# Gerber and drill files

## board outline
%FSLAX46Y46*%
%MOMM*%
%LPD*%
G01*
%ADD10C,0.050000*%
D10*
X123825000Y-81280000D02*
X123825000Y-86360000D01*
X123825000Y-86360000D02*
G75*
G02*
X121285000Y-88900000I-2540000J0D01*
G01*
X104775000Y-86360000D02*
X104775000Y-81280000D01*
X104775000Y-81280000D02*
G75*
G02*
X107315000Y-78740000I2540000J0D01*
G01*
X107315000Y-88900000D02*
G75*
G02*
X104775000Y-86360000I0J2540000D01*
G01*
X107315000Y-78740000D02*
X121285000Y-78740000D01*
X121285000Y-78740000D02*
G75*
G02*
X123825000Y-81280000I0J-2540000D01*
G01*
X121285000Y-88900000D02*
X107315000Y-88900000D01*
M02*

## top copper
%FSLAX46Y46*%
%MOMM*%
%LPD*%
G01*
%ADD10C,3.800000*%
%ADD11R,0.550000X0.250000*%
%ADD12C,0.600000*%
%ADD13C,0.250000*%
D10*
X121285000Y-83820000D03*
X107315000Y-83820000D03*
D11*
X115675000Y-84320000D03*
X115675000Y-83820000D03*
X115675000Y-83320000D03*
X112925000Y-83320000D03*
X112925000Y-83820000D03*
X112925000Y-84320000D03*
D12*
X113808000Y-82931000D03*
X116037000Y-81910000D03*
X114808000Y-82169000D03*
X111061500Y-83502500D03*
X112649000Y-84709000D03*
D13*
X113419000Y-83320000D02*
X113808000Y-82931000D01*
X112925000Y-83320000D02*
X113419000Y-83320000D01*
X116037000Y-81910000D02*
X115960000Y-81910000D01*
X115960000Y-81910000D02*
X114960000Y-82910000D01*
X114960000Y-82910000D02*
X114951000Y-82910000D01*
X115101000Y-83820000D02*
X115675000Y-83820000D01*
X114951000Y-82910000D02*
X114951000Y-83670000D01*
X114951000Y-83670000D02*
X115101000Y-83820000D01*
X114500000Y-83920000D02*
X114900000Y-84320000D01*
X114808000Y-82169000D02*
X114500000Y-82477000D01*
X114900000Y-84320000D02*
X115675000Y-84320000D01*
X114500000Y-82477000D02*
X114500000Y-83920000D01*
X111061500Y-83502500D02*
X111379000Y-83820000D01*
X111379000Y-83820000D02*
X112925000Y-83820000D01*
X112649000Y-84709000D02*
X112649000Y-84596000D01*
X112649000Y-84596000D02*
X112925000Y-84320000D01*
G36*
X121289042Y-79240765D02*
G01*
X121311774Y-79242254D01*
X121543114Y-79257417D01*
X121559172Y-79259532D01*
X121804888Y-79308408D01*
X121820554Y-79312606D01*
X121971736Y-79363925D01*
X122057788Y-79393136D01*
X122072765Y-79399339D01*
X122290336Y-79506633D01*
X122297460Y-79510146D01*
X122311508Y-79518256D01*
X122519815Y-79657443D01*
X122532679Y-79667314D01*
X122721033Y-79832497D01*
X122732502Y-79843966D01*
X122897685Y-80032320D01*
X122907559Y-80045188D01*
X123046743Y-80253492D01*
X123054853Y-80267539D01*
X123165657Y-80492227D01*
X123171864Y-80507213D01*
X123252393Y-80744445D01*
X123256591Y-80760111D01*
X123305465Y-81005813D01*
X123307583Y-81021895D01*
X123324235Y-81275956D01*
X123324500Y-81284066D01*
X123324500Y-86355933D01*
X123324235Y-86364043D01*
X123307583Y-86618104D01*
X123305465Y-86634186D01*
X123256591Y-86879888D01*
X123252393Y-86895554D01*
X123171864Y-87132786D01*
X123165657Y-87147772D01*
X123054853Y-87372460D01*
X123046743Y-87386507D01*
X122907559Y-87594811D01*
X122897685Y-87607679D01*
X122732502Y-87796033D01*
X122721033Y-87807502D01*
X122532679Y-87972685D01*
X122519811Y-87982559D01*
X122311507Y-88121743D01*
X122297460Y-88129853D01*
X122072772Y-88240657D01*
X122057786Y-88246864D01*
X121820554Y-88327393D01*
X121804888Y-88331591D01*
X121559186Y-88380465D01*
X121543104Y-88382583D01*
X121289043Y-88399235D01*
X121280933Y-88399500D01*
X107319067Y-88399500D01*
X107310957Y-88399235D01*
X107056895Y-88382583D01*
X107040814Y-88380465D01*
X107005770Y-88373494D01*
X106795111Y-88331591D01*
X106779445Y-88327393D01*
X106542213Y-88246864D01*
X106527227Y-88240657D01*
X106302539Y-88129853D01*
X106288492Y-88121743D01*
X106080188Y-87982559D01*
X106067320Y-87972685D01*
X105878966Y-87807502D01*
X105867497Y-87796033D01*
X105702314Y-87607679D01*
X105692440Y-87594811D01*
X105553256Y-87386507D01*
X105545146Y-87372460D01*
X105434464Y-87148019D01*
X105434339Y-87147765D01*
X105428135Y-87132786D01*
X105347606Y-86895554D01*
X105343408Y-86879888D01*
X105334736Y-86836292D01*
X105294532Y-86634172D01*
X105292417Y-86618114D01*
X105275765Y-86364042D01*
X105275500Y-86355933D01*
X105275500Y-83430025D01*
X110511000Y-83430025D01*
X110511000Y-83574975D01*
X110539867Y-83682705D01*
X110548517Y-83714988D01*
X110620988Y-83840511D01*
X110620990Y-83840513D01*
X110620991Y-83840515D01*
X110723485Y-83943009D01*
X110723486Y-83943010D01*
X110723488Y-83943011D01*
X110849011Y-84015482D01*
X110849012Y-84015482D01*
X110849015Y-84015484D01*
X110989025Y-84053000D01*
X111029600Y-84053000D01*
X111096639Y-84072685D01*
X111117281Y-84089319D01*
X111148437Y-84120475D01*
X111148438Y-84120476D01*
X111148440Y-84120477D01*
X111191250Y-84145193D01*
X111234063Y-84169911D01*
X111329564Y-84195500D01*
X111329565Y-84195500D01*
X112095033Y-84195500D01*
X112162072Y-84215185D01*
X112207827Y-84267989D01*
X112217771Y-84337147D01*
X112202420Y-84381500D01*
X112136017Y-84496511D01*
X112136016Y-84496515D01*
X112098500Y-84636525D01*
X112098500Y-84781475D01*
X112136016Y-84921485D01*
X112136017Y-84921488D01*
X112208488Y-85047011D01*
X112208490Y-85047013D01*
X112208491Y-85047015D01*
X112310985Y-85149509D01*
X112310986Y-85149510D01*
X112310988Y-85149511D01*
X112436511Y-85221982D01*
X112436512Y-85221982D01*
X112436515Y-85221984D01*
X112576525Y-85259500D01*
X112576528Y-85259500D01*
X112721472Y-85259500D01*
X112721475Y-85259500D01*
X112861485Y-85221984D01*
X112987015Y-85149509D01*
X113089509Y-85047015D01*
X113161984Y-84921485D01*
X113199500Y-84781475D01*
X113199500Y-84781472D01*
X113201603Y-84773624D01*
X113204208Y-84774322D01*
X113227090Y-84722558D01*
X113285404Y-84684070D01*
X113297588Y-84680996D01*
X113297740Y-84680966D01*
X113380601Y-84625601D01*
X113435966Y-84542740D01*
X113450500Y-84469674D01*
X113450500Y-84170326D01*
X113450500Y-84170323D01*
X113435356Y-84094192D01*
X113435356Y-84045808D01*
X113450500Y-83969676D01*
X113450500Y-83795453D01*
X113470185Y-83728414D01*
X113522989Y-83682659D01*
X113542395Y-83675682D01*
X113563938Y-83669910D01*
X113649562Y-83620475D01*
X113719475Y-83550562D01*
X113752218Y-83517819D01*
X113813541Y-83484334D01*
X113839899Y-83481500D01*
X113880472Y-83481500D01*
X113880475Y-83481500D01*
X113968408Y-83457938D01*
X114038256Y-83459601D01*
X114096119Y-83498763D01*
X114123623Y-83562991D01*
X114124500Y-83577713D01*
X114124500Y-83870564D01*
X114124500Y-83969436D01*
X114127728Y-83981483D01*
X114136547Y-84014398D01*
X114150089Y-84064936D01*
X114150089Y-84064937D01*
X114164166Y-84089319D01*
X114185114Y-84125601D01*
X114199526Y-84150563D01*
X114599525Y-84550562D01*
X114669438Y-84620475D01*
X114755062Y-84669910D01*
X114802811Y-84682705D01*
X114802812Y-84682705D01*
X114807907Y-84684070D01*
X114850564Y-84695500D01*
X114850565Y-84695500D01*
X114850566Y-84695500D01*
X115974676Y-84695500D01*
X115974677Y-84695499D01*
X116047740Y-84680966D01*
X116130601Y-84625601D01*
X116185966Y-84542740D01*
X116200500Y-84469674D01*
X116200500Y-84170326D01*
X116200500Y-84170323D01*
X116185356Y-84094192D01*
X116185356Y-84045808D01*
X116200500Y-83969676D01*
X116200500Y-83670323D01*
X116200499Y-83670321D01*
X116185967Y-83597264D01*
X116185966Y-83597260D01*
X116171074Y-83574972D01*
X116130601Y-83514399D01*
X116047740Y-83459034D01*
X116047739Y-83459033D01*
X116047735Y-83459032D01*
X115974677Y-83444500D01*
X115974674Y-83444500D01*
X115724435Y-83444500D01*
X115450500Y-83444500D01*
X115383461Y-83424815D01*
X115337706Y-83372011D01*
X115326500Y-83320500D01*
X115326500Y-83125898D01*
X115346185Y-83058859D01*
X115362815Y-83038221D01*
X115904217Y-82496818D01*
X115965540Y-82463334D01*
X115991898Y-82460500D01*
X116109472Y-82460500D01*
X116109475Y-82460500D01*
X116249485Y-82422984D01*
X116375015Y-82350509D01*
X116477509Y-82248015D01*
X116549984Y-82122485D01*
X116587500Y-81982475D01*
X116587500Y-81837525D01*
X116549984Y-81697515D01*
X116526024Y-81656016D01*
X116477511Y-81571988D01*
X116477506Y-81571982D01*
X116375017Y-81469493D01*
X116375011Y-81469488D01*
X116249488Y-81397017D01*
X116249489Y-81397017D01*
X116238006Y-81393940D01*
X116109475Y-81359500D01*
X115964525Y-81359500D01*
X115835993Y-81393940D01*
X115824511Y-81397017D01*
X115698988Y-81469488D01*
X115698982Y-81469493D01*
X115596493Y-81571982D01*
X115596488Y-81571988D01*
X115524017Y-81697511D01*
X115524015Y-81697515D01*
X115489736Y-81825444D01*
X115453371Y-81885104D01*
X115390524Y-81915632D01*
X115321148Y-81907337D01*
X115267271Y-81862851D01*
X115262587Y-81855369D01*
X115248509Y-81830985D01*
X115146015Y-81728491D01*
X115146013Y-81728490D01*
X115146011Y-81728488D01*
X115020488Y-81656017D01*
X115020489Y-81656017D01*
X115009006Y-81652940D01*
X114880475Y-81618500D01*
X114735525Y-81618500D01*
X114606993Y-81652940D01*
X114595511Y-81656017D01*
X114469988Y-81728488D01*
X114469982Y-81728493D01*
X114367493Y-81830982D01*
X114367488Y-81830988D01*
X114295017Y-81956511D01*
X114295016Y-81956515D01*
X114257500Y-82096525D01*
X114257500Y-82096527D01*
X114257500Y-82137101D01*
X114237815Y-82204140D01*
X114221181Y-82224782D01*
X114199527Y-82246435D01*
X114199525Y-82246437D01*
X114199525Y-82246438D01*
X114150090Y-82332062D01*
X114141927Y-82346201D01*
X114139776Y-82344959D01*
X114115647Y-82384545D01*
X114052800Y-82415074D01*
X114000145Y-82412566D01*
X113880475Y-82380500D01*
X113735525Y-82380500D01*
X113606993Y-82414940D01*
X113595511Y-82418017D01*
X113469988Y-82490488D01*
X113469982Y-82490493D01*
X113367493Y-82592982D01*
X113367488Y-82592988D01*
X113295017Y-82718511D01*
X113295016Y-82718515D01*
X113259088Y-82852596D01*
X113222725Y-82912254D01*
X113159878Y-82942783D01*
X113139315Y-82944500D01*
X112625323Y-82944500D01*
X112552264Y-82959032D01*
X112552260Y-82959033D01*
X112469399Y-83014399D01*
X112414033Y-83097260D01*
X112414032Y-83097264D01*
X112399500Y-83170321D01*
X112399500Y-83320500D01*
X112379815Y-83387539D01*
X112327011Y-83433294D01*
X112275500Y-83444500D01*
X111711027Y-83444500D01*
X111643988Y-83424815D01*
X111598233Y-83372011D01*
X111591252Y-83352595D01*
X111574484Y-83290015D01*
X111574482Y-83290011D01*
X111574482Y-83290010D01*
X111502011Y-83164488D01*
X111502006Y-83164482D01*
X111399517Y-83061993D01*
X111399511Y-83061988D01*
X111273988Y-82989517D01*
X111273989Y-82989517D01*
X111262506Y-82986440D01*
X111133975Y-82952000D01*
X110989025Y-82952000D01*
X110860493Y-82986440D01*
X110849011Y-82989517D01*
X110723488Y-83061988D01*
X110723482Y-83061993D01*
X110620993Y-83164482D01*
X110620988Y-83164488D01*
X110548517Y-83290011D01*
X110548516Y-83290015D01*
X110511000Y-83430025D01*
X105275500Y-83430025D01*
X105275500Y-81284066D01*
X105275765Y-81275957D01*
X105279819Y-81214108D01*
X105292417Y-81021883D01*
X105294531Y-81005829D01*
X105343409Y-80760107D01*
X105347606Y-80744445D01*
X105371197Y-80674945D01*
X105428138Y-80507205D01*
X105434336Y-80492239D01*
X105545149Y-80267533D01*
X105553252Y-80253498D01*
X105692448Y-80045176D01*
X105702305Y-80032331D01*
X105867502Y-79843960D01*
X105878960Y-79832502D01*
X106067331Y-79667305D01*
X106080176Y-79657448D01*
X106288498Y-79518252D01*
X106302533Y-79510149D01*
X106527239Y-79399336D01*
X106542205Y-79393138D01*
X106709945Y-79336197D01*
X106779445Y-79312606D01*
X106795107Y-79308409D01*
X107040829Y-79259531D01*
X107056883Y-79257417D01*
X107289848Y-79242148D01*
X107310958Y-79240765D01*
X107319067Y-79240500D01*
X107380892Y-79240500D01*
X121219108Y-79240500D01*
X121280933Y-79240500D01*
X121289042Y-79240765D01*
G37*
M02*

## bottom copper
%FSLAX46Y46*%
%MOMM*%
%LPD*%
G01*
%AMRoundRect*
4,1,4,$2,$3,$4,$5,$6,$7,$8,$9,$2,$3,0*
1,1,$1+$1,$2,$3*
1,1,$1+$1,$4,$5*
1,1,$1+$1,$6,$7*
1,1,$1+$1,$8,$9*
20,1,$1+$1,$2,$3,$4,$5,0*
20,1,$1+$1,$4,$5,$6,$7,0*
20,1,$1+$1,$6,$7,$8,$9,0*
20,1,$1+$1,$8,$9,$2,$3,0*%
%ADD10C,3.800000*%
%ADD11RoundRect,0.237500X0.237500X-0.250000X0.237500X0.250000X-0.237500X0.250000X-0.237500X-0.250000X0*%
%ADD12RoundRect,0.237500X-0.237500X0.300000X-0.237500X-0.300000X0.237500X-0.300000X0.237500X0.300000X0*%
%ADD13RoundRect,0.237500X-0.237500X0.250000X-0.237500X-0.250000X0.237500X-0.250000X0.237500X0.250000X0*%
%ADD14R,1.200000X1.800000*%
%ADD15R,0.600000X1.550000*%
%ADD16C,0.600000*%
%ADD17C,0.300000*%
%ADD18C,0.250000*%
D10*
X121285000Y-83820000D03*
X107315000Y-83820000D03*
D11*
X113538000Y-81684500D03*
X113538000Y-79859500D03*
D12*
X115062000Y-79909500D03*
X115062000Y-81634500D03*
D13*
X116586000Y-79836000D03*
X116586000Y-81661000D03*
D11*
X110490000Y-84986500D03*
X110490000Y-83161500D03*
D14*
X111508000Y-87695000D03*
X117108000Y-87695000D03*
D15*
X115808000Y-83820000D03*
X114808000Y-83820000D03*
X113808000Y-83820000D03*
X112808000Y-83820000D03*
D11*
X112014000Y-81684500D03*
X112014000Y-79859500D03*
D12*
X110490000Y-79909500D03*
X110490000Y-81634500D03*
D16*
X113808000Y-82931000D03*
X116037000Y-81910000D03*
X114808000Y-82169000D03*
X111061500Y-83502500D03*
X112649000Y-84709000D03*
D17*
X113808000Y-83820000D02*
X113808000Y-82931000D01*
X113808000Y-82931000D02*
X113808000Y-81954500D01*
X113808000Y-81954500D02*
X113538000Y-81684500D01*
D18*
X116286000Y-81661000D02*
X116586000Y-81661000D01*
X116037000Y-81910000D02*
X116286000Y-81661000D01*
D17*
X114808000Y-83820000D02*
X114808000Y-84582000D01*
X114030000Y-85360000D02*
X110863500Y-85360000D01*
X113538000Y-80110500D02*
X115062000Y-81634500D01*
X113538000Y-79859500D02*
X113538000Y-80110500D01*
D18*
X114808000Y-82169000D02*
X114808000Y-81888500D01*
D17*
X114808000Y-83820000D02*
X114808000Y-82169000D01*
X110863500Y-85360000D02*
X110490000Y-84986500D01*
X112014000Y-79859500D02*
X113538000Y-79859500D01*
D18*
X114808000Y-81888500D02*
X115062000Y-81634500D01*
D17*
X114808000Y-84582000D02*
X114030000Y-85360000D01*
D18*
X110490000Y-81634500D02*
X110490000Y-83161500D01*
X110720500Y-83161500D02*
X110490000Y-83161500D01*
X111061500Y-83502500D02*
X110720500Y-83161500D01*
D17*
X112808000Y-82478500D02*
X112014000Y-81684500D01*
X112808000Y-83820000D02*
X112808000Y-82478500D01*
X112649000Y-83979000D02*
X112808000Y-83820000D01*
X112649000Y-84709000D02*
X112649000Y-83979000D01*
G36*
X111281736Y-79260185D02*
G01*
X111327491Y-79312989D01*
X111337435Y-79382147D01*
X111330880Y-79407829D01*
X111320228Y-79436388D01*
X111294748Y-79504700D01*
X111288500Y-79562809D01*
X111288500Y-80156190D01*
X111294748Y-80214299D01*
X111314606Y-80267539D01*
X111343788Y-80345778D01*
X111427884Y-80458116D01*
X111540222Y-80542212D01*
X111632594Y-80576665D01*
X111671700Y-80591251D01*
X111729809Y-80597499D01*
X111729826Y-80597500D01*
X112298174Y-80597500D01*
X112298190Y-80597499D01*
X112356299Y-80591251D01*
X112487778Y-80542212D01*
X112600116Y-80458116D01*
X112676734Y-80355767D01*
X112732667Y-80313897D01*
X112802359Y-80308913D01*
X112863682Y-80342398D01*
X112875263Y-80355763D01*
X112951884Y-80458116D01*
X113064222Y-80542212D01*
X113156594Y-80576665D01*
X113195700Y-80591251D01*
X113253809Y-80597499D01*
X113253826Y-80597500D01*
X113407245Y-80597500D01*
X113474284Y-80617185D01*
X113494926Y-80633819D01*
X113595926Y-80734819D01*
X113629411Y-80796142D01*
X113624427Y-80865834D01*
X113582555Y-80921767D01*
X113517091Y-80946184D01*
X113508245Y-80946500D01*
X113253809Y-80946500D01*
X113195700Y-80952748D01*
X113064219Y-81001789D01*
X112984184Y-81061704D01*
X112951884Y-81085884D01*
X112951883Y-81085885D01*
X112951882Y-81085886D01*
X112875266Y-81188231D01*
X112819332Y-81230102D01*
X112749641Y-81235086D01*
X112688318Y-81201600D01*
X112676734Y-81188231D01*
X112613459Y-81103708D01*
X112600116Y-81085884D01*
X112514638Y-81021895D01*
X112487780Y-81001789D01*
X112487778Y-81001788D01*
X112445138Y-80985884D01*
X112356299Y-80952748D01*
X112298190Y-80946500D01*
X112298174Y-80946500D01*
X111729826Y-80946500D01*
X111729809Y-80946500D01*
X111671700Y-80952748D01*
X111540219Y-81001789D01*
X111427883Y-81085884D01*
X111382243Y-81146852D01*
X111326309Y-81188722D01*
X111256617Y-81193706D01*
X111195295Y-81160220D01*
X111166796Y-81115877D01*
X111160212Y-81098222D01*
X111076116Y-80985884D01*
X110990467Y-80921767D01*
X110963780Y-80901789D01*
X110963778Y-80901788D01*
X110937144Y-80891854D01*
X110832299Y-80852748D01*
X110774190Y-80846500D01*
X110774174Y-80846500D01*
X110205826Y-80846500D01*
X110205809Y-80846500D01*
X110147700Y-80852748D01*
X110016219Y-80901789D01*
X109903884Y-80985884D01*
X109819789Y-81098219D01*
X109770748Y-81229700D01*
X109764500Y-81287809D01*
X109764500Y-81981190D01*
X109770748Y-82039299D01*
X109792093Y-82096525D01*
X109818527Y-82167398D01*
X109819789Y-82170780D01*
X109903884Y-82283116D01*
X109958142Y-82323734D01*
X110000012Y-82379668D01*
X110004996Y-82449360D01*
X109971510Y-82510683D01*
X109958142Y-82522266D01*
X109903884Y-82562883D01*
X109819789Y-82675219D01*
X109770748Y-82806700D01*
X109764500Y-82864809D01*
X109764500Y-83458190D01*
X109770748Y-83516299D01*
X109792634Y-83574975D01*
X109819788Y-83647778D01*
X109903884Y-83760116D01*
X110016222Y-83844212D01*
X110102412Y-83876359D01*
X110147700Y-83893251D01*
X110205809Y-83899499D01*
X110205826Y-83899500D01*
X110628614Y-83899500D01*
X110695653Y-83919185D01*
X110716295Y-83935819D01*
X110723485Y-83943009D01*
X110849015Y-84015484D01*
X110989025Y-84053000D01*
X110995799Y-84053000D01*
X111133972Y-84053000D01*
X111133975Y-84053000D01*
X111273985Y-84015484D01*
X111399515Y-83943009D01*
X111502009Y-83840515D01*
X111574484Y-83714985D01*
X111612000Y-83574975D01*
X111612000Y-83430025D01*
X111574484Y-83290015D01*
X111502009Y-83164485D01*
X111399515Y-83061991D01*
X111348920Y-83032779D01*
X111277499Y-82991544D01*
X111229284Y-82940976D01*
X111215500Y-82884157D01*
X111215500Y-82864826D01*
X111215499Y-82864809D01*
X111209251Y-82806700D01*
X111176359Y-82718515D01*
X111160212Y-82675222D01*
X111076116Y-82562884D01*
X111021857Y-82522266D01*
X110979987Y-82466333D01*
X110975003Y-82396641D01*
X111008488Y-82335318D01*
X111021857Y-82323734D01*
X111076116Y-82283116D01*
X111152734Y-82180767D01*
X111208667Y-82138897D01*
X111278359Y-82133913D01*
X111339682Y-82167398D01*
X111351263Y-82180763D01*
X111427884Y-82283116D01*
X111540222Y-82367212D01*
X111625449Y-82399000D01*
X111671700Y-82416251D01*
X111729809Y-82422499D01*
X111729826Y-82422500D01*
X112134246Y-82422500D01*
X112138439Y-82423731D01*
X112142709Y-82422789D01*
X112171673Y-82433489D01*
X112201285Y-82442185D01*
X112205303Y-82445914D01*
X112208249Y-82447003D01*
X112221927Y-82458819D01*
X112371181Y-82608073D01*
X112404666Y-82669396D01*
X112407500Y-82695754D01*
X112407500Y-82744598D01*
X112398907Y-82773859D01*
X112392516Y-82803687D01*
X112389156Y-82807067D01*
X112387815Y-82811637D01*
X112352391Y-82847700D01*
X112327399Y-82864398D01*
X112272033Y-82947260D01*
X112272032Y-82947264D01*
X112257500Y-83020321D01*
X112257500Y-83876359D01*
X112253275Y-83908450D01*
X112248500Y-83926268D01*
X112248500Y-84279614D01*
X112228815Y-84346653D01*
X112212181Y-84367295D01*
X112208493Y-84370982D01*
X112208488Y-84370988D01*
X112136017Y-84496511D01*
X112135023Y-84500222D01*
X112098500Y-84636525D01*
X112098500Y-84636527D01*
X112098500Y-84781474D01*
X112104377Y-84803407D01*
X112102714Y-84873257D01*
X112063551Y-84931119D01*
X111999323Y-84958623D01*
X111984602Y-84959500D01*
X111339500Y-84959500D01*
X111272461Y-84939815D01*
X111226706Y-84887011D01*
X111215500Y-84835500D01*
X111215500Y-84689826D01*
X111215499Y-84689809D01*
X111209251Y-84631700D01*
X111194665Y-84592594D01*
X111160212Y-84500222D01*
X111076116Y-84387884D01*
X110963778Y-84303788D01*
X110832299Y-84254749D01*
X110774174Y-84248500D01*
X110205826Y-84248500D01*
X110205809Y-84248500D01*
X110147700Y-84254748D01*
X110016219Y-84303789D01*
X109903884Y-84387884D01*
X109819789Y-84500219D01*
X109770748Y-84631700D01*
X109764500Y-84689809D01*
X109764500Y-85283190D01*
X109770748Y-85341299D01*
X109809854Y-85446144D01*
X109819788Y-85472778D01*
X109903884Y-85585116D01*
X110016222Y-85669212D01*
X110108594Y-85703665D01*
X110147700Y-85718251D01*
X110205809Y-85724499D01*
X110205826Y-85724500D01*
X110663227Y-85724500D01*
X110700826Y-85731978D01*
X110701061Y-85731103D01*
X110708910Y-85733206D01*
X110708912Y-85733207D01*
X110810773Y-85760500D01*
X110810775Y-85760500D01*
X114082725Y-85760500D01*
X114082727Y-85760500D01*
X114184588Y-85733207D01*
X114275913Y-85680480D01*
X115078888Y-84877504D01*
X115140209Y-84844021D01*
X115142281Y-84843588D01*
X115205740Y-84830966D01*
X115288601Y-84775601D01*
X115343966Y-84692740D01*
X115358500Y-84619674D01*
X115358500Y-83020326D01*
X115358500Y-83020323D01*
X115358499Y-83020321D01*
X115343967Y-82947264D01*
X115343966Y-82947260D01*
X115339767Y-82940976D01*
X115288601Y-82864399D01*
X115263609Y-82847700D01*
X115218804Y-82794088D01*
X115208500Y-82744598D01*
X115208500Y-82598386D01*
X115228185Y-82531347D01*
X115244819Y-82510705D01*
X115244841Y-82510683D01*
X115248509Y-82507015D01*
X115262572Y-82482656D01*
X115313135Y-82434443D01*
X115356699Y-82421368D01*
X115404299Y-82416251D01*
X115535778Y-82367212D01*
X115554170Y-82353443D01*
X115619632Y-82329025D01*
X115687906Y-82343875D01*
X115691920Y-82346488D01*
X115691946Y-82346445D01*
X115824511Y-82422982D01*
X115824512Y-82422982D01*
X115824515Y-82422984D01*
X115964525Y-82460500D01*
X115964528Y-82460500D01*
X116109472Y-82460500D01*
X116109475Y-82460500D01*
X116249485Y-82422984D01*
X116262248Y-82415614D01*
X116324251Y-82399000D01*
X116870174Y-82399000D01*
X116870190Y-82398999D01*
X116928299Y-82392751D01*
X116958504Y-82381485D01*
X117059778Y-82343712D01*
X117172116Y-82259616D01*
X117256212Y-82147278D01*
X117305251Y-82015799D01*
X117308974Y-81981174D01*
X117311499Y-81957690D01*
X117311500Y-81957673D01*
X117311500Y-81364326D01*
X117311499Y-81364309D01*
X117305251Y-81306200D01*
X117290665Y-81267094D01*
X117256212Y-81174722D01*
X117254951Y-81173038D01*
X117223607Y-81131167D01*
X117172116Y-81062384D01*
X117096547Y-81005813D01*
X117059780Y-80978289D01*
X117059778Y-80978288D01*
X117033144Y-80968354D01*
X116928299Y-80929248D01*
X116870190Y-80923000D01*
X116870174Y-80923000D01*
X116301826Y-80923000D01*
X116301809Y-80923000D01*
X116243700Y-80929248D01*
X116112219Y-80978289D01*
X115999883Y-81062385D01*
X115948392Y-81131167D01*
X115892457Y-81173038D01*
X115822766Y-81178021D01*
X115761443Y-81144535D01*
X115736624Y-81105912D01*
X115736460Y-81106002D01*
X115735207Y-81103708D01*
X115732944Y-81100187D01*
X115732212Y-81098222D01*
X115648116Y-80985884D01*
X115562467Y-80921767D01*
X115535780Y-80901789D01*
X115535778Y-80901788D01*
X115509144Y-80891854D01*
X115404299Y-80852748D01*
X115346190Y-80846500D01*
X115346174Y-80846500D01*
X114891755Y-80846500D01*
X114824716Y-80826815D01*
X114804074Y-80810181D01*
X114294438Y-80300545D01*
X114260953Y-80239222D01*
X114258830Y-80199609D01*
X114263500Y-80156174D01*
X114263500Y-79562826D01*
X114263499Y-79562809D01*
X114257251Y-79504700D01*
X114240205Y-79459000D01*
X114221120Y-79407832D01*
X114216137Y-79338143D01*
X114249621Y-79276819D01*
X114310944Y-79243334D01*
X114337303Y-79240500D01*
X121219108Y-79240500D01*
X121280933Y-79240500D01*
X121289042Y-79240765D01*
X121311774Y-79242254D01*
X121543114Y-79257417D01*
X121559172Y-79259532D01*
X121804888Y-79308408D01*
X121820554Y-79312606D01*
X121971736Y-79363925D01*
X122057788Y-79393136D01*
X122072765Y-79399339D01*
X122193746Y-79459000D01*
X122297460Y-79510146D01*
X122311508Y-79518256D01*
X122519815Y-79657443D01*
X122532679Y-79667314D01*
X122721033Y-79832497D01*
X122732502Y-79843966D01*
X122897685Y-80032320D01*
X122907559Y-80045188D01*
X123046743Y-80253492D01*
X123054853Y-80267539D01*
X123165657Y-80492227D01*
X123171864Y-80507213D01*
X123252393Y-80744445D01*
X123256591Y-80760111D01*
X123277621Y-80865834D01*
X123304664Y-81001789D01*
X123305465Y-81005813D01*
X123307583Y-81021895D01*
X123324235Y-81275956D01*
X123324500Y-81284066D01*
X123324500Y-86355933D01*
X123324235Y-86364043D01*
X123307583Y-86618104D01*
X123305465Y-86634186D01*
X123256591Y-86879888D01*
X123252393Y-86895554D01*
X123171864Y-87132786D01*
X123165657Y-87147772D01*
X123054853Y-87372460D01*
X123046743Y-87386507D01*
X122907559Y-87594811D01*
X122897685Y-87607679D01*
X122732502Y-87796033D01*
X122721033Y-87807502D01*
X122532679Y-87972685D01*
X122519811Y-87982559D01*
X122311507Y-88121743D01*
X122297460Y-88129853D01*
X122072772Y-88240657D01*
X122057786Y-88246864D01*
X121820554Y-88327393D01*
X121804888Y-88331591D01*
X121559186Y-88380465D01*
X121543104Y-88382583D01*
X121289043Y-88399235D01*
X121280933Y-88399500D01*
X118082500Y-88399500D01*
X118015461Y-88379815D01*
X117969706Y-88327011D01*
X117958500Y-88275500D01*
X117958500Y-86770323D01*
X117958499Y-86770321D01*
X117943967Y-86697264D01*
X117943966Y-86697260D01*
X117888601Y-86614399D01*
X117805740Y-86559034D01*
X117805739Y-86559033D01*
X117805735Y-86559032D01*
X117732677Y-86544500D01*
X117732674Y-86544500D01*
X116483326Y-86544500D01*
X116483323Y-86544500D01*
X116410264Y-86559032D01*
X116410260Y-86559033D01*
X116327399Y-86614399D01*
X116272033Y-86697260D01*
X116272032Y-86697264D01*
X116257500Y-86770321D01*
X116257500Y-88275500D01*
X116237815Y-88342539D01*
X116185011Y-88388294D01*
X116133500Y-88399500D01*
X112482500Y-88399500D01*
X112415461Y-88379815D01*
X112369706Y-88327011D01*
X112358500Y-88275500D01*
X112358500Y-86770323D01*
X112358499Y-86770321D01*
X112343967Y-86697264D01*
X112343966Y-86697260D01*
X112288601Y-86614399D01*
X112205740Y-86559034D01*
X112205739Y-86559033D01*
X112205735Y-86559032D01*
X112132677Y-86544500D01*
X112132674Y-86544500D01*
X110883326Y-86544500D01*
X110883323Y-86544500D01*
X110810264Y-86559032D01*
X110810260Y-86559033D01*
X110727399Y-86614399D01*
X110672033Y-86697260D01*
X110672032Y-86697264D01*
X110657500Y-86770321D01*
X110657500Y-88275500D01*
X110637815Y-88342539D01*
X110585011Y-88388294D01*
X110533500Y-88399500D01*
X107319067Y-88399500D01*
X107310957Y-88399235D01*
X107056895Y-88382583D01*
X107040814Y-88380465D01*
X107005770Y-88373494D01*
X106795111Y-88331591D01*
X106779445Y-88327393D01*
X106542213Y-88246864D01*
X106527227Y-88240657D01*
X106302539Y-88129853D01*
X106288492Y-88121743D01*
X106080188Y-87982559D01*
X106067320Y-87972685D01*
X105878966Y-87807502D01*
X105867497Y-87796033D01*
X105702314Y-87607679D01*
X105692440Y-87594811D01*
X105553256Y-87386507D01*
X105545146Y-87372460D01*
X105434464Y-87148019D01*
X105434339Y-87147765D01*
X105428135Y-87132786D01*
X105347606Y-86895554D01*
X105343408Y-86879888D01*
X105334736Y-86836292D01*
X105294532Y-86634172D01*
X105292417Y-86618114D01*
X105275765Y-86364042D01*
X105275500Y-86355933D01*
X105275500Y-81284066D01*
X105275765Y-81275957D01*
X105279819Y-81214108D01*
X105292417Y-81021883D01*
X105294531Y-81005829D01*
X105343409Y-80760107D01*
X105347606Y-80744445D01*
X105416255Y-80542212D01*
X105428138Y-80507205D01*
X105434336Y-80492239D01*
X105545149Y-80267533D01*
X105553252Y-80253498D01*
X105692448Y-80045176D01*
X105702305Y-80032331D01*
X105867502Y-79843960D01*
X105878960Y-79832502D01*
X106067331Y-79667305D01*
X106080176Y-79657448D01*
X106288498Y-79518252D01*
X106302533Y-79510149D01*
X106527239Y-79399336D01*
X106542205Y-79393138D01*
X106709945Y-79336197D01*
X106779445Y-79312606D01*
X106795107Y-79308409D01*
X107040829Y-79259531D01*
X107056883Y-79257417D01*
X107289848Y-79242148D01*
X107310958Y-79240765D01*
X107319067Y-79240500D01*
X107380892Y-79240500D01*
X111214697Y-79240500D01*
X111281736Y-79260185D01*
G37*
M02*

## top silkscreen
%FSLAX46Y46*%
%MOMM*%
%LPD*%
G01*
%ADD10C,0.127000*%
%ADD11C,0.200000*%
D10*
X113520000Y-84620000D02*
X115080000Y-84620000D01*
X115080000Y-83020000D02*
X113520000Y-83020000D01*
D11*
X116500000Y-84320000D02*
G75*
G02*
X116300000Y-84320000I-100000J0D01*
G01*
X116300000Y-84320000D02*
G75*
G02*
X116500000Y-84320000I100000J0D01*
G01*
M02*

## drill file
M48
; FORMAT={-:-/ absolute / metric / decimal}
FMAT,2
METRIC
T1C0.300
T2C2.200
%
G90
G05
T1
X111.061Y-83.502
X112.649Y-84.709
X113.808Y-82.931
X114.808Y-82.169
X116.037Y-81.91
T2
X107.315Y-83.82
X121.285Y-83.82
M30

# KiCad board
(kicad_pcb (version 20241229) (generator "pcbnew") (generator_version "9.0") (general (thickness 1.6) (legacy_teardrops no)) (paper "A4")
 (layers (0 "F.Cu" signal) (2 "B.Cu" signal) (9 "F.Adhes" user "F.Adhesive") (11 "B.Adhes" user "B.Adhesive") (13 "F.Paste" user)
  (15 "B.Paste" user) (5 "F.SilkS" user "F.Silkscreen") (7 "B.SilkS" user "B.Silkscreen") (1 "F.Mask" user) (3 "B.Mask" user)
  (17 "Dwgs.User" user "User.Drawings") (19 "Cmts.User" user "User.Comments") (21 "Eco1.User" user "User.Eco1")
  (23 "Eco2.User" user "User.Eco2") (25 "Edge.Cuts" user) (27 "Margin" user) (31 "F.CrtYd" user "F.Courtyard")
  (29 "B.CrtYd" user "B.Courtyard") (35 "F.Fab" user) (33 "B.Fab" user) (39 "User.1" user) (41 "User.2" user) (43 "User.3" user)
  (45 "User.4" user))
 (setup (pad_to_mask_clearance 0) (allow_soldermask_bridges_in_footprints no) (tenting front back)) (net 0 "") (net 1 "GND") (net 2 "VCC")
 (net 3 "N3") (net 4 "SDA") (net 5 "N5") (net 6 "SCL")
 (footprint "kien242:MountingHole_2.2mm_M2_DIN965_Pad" (layer "F.Cu") (at 121.285 83.82)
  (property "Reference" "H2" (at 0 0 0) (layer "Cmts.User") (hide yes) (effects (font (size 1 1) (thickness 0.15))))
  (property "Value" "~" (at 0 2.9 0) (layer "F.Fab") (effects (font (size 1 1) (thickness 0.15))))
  (pad "1" thru_hole circle (at 0 0) (size 3.8 3.8) (drill 2.2) (layers "*.Cu" "*.Mask") (remove_unused_layers no) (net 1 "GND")))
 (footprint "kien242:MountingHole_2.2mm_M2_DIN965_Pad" (layer "F.Cu") (at 107.315 83.82)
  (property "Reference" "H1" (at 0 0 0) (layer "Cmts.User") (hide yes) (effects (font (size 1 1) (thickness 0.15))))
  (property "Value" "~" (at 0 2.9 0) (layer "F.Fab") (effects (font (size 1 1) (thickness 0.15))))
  (pad "1" thru_hole circle (at 0 0) (size 3.8 3.8) (drill 2.2) (layers "*.Cu" "*.Mask") (remove_unused_layers no) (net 1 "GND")))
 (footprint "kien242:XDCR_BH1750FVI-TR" (layer "F.Cu") (at 114.3 83.82 180)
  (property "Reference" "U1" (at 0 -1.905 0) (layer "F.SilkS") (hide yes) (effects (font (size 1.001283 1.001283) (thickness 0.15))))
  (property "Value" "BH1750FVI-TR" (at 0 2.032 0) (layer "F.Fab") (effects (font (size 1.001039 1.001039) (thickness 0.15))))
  (fp_line (start 0.78 -0.8) (end -0.78 -0.8) (stroke (width 0.127) (type solid)) (layer "F.SilkS"))
  (fp_line (start -0.78 0.8) (end 0.78 0.8) (stroke (width 0.127) (type solid)) (layer "F.SilkS"))
  (fp_circle (center -2.1 -0.5) (end -2 -0.5) (stroke (width 0.2) (type solid)) (fill no) (layer "F.SilkS"))
  (pad "1" smd rect (at -1.375 -0.5 180) (size 0.55 0.25) (layers "F.Cu" "F.Mask" "F.Paste") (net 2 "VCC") (solder_mask_margin 0.102))
  (pad "2" smd rect (at -1.375 0 180) (size 0.55 0.25) (layers "F.Cu" "F.Mask" "F.Paste") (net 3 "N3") (solder_mask_margin 0.102))
  (pad "3" smd rect (at -1.375 0.5 180) (size 0.55 0.25) (layers "F.Cu" "F.Mask" "F.Paste") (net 1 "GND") (solder_mask_margin 0.102))
  (pad "4" smd rect (at 1.375 0.5 180) (size 0.55 0.25) (layers "F.Cu" "F.Mask" "F.Paste") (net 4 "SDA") (solder_mask_margin 0.102))
  (pad "5" smd rect (at 1.375 0 180) (size 0.55 0.25) (layers "F.Cu" "F.Mask" "F.Paste") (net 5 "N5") (solder_mask_margin 0.102))
  (pad "6" smd rect (at 1.375 -0.5 180) (size 0.55 0.25) (layers "F.Cu" "F.Mask" "F.Paste") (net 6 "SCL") (solder_mask_margin 0.102)))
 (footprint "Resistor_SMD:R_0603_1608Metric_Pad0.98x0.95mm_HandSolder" (layer "B.Cu") (at 113.538 80.772 90)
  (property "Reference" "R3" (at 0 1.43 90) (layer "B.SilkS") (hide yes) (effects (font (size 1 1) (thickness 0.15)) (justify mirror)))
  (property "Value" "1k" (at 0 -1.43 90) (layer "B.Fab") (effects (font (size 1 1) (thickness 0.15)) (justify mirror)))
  (pad "1" smd roundrect (at -0.9125 0 90) (size 0.975 0.95) (layers "B.Cu" "B.Mask" "B.Paste") (roundrect_rratio 0.25) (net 4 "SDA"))
  (pad "2" smd roundrect (at 0.9125 0 90) (size 0.975 0.95) (layers "B.Cu" "B.Mask" "B.Paste") (roundrect_rratio 0.25) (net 2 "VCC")))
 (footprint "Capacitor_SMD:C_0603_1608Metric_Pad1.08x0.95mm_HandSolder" (layer "B.Cu") (at 115.062 80.772 -90)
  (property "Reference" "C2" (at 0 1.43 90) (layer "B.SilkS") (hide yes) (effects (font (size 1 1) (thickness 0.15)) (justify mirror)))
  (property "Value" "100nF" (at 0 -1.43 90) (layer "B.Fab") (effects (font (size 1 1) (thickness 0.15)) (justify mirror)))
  (pad "1" smd roundrect (at -0.8625 0 270) (size 1.075 0.95) (layers "B.Cu" "B.Mask" "B.Paste") (roundrect_rratio 0.25) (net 1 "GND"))
  (pad "2" smd roundrect (at 0.8625 0 270) (size 1.075 0.95) (layers "B.Cu" "B.Mask" "B.Paste") (roundrect_rratio 0.25) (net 2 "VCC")))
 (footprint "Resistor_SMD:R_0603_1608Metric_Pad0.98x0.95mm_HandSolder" (layer "B.Cu") (at 116.586 80.7485 -90)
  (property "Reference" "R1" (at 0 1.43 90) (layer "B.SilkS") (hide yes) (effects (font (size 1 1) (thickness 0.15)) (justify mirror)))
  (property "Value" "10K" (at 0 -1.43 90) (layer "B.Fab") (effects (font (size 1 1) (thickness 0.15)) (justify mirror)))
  (pad "1" smd roundrect (at -0.9125 0 270) (size 0.975 0.95) (layers "B.Cu" "B.Mask" "B.Paste") (roundrect_rratio 0.25) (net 1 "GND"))
  (pad "2" smd roundrect (at 0.9125 0 270) (size 0.975 0.95) (layers "B.Cu" "B.Mask" "B.Paste") (roundrect_rratio 0.25) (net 3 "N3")))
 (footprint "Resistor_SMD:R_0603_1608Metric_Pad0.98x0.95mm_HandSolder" (layer "B.Cu") (at 110.49 84.074 90)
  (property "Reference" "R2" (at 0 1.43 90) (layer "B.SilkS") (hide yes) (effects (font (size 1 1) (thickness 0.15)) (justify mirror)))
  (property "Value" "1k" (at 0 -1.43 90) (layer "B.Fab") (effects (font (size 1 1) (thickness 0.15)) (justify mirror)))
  (pad "1" smd roundrect (at -0.9125 0 90) (size 0.975 0.95) (layers "B.Cu" "B.Mask" "B.Paste") (roundrect_rratio 0.25) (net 2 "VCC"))
  (pad "2" smd roundrect (at 0.9125 0 90) (size 0.975 0.95) (layers "B.Cu" "B.Mask" "B.Paste") (roundrect_rratio 0.25) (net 5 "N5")))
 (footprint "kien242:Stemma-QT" (layer "B.Cu") (at 114.3 86.36 90)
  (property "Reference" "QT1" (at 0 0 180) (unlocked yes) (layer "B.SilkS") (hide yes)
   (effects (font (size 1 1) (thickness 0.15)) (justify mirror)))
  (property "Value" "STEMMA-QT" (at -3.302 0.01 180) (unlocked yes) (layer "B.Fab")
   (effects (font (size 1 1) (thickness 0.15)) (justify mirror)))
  (pad "" smd rect (at -1.335 -2.792 180) (size 1.2 1.8) (layers "B.Cu" "B.Mask" "B.Paste"))
  (pad "" smd rect (at -1.335 2.808 180) (size 1.2 1.8) (layers "B.Cu" "B.Mask" "B.Paste"))
  (pad "1" smd rect (at 2.54 1.508 180) (size 0.6 1.55) (layers "B.Cu" "B.Mask" "B.Paste") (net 1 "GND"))
  (pad "2" smd rect (at 2.54 0.508 180) (size 0.6 1.55) (layers "B.Cu" "B.Mask" "B.Paste") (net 2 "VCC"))
  (pad "3" smd rect (at 2.54 -0.492 180) (size 0.6 1.55) (layers "B.Cu" "B.Mask" "B.Paste") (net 4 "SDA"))
  (pad "4" smd rect (at 2.54 -1.492 180) (size 0.6 1.55) (layers "B.Cu" "B.Mask" "B.Paste") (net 6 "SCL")))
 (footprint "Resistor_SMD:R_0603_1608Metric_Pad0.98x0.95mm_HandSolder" (layer "B.Cu") (at 112.014 80.772 90)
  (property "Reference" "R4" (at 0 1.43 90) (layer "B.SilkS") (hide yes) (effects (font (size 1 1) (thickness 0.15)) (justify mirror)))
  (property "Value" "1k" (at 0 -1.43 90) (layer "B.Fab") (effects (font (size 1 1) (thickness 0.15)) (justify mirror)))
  (pad "1" smd roundrect (at -0.9125 0 90) (size 0.975 0.95) (layers "B.Cu" "B.Mask" "B.Paste") (roundrect_rratio 0.25) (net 6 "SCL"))
  (pad "2" smd roundrect (at 0.9125 0 90) (size 0.975 0.95) (layers "B.Cu" "B.Mask" "B.Paste") (roundrect_rratio 0.25) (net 2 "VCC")))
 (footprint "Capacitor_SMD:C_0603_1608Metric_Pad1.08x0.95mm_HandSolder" (layer "B.Cu") (at 110.49 80.772 -90)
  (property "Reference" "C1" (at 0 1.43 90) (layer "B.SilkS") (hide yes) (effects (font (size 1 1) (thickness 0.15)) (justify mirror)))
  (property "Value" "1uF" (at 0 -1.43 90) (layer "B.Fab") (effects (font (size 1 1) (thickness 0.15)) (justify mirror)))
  (pad "1" smd roundrect (at -0.8625 0 270) (size 1.075 0.95) (layers "B.Cu" "B.Mask" "B.Paste") (roundrect_rratio 0.25) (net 1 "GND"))
  (pad "2" smd roundrect (at 0.8625 0 270) (size 1.075 0.95) (layers "B.Cu" "B.Mask" "B.Paste") (roundrect_rratio 0.25) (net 5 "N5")))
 (gr_line (start 123.825 81.28) (end 123.825 86.36) (stroke (width 0.05) (type default)) (layer "Edge.Cuts"))
 (gr_arc (start 123.825 86.36) (mid 123.081051 88.156051) (end 121.285 88.9) (stroke (width 0.05) (type default)) (layer "Edge.Cuts"))
 (gr_line (start 104.775 86.36) (end 104.775 81.28) (stroke (width 0.05) (type default)) (layer "Edge.Cuts"))
 (gr_arc (start 104.775 81.28) (mid 105.518949 79.483949) (end 107.315 78.74) (stroke (width 0.05) (type default)) (layer "Edge.Cuts"))
 (gr_arc (start 107.315 88.9) (mid 105.518949 88.156051) (end 104.775 86.36) (stroke (width 0.05) (type default)) (layer "Edge.Cuts"))
 (gr_line (start 107.315 78.74) (end 121.285 78.74) (stroke (width 0.05) (type default)) (layer "Edge.Cuts"))
 (gr_arc (start 121.285 78.74) (mid 123.081051 79.483949) (end 123.825 81.28) (stroke (width 0.05) (type default)) (layer "Edge.Cuts"))
 (gr_line (start 121.285 88.9) (end 107.315 88.9) (stroke (width 0.05) (type default)) (layer "Edge.Cuts"))
 (segment (start 113.419 83.32) (end 113.808 82.931) (width 0.25) (layer "F.Cu") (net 4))
 (segment (start 112.925 83.32) (end 113.419 83.32) (width 0.25) (layer "F.Cu") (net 4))
 (via (at 113.808 82.931) (size 0.6) (drill 0.3) (layers "F.Cu" "B.Cu") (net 4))
 (segment (start 113.808 83.82) (end 113.808 82.931) (width 0.3) (layer "B.Cu") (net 4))
 (segment (start 113.808 82.931) (end 113.808 81.9545) (width 0.3) (layer "B.Cu") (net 4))
 (segment (start 113.808 81.9545) (end 113.538 81.6845) (width 0.3) (layer "B.Cu") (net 4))
 (segment (start 116.037 81.91) (end 115.96 81.91) (width 0.25) (layer "F.Cu") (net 3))
 (segment (start 115.96 81.91) (end 114.96 82.91) (width 0.25) (layer "F.Cu") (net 3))
 (segment (start 114.96 82.91) (end 114.951 82.91) (width 0.25) (layer "F.Cu") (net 3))
 (segment (start 115.101 83.82) (end 115.675 83.82) (width 0.25) (layer "F.Cu") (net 3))
 (segment (start 114.951 82.91) (end 114.951 83.67) (width 0.25) (layer "F.Cu") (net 3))
 (segment (start 114.951 83.67) (end 115.101 83.82) (width 0.25) (layer "F.Cu") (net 3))
 (via (at 116.037 81.91) (size 0.6) (drill 0.3) (layers "F.Cu" "B.Cu") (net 3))
 (segment (start 116.286 81.661) (end 116.586 81.661) (width 0.25) (layer "B.Cu") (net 3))
 (segment (start 116.037 81.91) (end 116.286 81.661) (width 0.25) (layer "B.Cu") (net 3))
 (segment (start 114.5 83.92) (end 114.9 84.32) (width 0.25) (layer "F.Cu") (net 2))
 (segment (start 114.808 82.169) (end 114.5 82.477) (width 0.25) (layer "F.Cu") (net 2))
 (segment (start 114.9 84.32) (end 115.675 84.32) (width 0.25) (layer "F.Cu") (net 2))
 (segment (start 114.5 82.477) (end 114.5 83.92) (width 0.25) (layer "F.Cu") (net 2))
 (via (at 114.808 82.169) (size 0.6) (drill 0.3) (layers "F.Cu" "B.Cu") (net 2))
 (segment (start 114.808 83.82) (end 114.808 84.582) (width 0.3) (layer "B.Cu") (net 2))
 (segment (start 114.03 85.36) (end 110.8635 85.36) (width 0.3) (layer "B.Cu") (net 2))
 (segment (start 113.538 80.1105) (end 115.062 81.6345) (width 0.3) (layer "B.Cu") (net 2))
 (segment (start 113.538 79.8595) (end 113.538 80.1105) (width 0.3) (layer "B.Cu") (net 2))
 (segment (start 114.808 82.169) (end 114.808 81.8885) (width 0.25) (layer "B.Cu") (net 2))
 (segment (start 114.808 83.82) (end 114.808 82.169) (width 0.3) (layer "B.Cu") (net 2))
 (segment (start 110.8635 85.36) (end 110.49 84.9865) (width 0.3) (layer "B.Cu") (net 2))
 (segment (start 112.014 79.8595) (end 113.538 79.8595) (width 0.3) (layer "B.Cu") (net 2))
 (segment (start 114.808 81.8885) (end 115.062 81.6345) (width 0.25) (layer "B.Cu") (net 2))
 (segment (start 114.808 84.582) (end 114.03 85.36) (width 0.3) (layer "B.Cu") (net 2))
 (segment (start 111.0615 83.5025) (end 111.379 83.82) (width 0.25) (layer "F.Cu") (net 5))
 (segment (start 111.379 83.82) (end 112.925 83.82) (width 0.25) (layer "F.Cu") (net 5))
 (via (at 111.0615 83.5025) (size 0.6) (drill 0.3) (layers "F.Cu" "B.Cu") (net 5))
 (segment (start 110.49 81.6345) (end 110.49 83.1615) (width 0.25) (layer "B.Cu") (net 5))
 (segment (start 110.7205 83.1615) (end 110.49 83.1615) (width 0.25) (layer "B.Cu") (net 5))
 (segment (start 111.0615 83.5025) (end 110.7205 83.1615) (width 0.25) (layer "B.Cu") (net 5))
 (segment (start 112.649 84.709) (end 112.649 84.596) (width 0.25) (layer "F.Cu") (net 6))
 (segment (start 112.649 84.596) (end 112.925 84.32) (width 0.25) (layer "F.Cu") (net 6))
 (via (at 112.649 84.709) (size 0.6) (drill 0.3) (layers "F.Cu" "B.Cu") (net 6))
 (segment (start 112.808 82.4785) (end 112.014 81.6845) (width 0.3) (layer "B.Cu") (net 6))
 (segment (start 112.808 83.82) (end 112.808 82.4785) (width 0.3) (layer "B.Cu") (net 6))
 (segment (start 112.649 83.979) (end 112.808 83.82) (width 0.3) (layer "B.Cu") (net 6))
 (segment (start 112.649 84.709) (end 112.649 83.979) (width 0.3) (layer "B.Cu") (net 6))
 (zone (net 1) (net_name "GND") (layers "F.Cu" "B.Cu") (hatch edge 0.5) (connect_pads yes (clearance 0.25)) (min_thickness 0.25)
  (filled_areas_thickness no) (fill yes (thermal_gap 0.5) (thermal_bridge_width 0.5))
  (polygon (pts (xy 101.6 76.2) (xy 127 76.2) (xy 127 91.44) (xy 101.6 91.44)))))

